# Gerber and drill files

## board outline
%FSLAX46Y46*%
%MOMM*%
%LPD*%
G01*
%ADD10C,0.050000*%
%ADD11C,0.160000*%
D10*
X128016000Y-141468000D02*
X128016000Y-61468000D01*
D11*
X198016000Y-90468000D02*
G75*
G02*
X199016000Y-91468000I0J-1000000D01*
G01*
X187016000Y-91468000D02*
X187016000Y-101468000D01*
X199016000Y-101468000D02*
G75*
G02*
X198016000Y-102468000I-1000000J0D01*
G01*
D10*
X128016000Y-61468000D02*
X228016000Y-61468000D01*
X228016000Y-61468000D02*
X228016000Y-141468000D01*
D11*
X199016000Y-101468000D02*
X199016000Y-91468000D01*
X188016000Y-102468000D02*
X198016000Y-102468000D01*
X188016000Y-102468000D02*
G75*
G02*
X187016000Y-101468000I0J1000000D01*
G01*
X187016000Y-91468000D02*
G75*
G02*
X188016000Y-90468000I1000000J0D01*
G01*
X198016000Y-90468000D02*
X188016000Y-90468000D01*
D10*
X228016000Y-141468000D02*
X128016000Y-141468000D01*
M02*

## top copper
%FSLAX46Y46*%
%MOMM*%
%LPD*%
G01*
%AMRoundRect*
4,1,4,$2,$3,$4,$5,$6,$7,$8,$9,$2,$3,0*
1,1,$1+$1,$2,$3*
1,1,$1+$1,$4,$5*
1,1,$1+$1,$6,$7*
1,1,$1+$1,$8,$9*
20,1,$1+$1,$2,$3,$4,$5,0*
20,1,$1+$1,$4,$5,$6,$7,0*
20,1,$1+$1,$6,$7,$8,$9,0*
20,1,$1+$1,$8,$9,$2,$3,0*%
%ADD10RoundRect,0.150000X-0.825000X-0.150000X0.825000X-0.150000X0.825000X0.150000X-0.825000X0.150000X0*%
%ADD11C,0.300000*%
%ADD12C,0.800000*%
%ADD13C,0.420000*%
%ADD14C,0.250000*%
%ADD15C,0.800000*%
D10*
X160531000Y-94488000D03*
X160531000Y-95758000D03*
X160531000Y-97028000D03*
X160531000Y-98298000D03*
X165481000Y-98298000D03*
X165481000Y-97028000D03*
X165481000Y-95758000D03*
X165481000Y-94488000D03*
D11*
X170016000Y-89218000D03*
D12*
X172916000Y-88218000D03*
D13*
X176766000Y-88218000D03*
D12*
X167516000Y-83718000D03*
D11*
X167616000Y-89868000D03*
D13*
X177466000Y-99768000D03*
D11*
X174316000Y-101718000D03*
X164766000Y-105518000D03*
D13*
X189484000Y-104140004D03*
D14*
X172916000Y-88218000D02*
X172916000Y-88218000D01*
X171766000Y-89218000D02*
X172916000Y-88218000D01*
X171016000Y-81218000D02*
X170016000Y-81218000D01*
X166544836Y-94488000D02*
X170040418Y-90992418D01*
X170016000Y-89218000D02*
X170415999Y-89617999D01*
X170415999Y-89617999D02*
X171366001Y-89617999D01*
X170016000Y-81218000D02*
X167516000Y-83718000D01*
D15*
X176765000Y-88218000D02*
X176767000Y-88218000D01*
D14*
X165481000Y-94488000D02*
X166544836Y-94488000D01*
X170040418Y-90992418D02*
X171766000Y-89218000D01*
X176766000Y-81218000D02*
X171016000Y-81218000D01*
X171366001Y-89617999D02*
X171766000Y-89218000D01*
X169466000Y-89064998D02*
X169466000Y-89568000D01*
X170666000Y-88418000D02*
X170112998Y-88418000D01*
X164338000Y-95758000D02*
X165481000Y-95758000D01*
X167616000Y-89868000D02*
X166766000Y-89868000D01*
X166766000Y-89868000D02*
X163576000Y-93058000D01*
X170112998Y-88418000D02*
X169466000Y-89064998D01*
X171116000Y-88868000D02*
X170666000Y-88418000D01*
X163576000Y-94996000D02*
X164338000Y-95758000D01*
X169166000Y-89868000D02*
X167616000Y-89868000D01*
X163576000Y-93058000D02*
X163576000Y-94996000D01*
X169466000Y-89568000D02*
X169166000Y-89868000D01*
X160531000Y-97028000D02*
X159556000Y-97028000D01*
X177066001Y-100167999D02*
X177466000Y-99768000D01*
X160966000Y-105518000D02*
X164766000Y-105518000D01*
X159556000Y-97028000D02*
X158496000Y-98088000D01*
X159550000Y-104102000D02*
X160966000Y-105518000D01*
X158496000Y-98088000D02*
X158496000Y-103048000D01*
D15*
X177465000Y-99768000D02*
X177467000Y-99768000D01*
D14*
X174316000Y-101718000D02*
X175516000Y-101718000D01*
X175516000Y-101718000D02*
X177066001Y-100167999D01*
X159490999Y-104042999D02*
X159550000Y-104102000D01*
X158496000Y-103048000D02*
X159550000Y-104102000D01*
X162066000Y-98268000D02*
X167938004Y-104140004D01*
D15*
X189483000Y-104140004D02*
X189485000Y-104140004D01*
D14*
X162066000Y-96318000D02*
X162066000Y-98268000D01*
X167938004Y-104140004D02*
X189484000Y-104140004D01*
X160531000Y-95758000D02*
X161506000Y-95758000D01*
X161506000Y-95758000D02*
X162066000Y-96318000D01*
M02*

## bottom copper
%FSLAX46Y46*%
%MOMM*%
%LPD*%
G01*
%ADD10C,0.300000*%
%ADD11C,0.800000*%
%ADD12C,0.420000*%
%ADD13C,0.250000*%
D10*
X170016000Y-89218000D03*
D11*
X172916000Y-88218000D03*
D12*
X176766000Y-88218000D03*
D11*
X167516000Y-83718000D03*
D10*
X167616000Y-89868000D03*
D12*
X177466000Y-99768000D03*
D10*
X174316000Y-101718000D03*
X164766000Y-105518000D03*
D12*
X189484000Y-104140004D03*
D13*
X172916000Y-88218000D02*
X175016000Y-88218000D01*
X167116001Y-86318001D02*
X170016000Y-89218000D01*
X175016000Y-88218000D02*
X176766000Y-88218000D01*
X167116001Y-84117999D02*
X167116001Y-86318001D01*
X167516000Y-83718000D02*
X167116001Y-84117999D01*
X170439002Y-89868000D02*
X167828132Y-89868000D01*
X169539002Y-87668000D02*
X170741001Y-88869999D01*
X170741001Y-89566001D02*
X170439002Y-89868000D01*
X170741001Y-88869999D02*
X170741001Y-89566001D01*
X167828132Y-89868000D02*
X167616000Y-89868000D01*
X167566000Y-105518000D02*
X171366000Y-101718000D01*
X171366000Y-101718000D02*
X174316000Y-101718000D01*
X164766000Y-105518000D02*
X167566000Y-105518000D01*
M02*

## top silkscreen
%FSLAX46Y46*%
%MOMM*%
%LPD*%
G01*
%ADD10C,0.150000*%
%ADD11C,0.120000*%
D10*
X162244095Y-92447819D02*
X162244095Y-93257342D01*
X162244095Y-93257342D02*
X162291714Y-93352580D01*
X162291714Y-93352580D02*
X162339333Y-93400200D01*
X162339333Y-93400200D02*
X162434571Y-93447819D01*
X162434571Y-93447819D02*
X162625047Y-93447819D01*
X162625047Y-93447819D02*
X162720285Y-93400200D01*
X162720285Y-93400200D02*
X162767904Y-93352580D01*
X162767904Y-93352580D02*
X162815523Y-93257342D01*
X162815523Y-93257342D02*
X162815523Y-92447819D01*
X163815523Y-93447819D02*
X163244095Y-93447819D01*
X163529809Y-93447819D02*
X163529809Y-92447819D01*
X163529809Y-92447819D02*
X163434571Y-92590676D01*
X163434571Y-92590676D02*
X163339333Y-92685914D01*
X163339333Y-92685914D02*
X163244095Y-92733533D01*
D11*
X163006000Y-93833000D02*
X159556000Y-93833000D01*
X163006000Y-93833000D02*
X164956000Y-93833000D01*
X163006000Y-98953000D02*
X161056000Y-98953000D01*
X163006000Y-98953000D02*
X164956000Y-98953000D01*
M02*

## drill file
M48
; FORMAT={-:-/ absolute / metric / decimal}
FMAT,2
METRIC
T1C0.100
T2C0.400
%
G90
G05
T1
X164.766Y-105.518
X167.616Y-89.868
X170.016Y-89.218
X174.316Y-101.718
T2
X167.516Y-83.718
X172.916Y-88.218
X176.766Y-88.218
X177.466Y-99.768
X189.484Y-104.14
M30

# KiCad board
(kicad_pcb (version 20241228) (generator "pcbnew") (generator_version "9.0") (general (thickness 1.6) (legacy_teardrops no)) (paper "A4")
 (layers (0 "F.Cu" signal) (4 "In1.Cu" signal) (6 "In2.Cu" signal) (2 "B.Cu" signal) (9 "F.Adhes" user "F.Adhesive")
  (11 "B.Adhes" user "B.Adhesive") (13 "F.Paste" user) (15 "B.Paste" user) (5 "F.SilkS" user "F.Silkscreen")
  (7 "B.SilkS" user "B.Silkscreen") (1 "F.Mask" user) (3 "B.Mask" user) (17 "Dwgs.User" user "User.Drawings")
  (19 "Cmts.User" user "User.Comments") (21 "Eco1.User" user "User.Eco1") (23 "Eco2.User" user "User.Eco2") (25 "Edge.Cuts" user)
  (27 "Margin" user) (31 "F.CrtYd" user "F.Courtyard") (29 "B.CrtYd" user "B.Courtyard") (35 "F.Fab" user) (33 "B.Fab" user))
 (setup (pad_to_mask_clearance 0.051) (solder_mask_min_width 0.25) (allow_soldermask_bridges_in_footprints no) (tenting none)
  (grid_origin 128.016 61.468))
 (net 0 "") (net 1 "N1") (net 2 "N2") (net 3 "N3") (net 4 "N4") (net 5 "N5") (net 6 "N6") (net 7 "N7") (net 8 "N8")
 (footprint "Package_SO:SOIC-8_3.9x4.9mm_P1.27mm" (layer "F.Cu") (at 163.006 96.393)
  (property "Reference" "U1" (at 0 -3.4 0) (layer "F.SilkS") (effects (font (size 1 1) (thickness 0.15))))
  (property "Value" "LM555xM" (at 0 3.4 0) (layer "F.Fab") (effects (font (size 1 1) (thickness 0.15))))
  (fp_line (start 0 -2.56) (end -3.45 -2.56) (stroke (width 0.12) (type solid)) (layer "F.SilkS"))
  (fp_line (start 0 -2.56) (end 1.95 -2.56) (stroke (width 0.12) (type solid)) (layer "F.SilkS"))
  (fp_line (start 0 2.56) (end -1.95 2.56) (stroke (width 0.12) (type solid)) (layer "F.SilkS"))
  (fp_line (start 0 2.56) (end 1.95 2.56) (stroke (width 0.12) (type solid)) (layer "F.SilkS"))
  (pad "1" smd roundrect (at -2.475 -1.905) (size 1.95 0.6) (layers "F.Cu" "F.Mask" "F.Paste") (roundrect_rratio 0.25) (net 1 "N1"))
  (pad "2" smd roundrect (at -2.475 -0.635) (size 1.95 0.6) (layers "F.Cu" "F.Mask" "F.Paste") (roundrect_rratio 0.25) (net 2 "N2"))
  (pad "3" smd roundrect (at -2.475 0.635) (size 1.95 0.6) (layers "F.Cu" "F.Mask" "F.Paste") (roundrect_rratio 0.25) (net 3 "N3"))
  (pad "4" smd roundrect (at -2.475 1.905) (size 1.95 0.6) (layers "F.Cu" "F.Mask" "F.Paste") (roundrect_rratio 0.25) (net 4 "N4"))
  (pad "5" smd roundrect (at 2.475 1.905) (size 1.95 0.6) (layers "F.Cu" "F.Mask" "F.Paste") (roundrect_rratio 0.25) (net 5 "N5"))
  (pad "6" smd roundrect (at 2.475 0.635) (size 1.95 0.6) (layers "F.Cu" "F.Mask" "F.Paste") (roundrect_rratio 0.25) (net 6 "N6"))
  (pad "7" smd roundrect (at 2.475 -0.635) (size 1.95 0.6) (layers "F.Cu" "F.Mask" "F.Paste") (roundrect_rratio 0.25) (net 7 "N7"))
  (pad "8" smd roundrect (at 2.475 -1.905) (size 1.95 0.6) (layers "F.Cu" "F.Mask" "F.Paste") (roundrect_rratio 0.25) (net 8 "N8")))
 (gr_line (start 128.016 141.468) (end 128.016 61.468) (stroke (width 0.05) (type solid)) (layer "Edge.Cuts"))
 (gr_arc (start 198.016 90.468) (mid 198.723107 90.760893) (end 199.016 91.468) (stroke (width 0.16) (type solid)) (layer "Edge.Cuts"))
 (gr_line (start 187.016 91.468) (end 187.016 101.468) (stroke (width 0.16) (type solid)) (layer "Edge.Cuts"))
 (gr_arc (start 199.016 101.468) (mid 198.723107 102.175107) (end 198.016 102.468) (stroke (width 0.16) (type solid)) (layer "Edge.Cuts"))
 (gr_line (start 128.016 61.468) (end 228.016 61.468) (stroke (width 0.05) (type solid)) (layer "Edge.Cuts"))
 (gr_line (start 228.016 61.468) (end 228.016 141.468) (stroke (width 0.05) (type solid)) (layer "Edge.Cuts"))
 (gr_line (start 199.016 101.468) (end 199.016 91.468) (stroke (width 0.16) (type solid)) (layer "Edge.Cuts"))
 (gr_line (start 188.016 102.468) (end 198.016 102.468) (stroke (width 0.16) (type solid)) (layer "Edge.Cuts"))
 (gr_arc (start 188.016 102.468) (mid 187.308893 102.175107) (end 187.016 101.468) (stroke (width 0.16) (type solid)) (layer "Edge.Cuts"))
 (gr_arc (start 187.016 91.468) (mid 187.308893 90.760893) (end 188.016 90.468) (stroke (width 0.16) (type solid)) (layer "Edge.Cuts"))
 (gr_line (start 198.016 90.468) (end 188.016 90.468) (stroke (width 0.16) (type solid)) (layer "Edge.Cuts"))
 (gr_line (start 228.016 141.468) (end 128.016 141.468) (stroke (width 0.05) (type solid)) (layer "Edge.Cuts"))
 (segment (start 172.916 88.218) (end 172.916 88.218) (width 0.25) (layer "F.Cu") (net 8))
 (segment (start 171.766 89.218) (end 172.916 88.218) (width 0.25) (layer "F.Cu") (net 8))
 (segment (start 171.016 81.218) (end 170.016 81.218) (width 0.25) (layer "F.Cu") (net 8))
 (segment (start 166.544836 94.488) (end 170.040418 90.992418) (width 0.25) (layer "F.Cu") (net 8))
 (segment (start 170.016 89.218) (end 170.415999 89.617999) (width 0.25) (layer "F.Cu") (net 8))
 (segment (start 170.415999 89.617999) (end 171.366001 89.617999) (width 0.25) (layer "F.Cu") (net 8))
 (segment (start 170.016 81.218) (end 167.516 83.718) (width 0.25) (layer "F.Cu") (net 8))
 (segment (start 176.765 88.218) (end 176.767 88.218) (width 0.8) (layer "F.Cu") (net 8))
 (segment (start 165.481 94.488) (end 166.544836 94.488) (width 0.25) (layer "F.Cu") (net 8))
 (segment (start 170.040418 90.992418) (end 171.766 89.218) (width 0.25) (layer "F.Cu") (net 8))
 (segment (start 176.766 81.218) (end 171.016 81.218) (width 0.25) (layer "F.Cu") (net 8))
 (segment (start 171.366001 89.617999) (end 171.766 89.218) (width 0.25) (layer "F.Cu") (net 8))
 (via (at 170.016 89.218) (size 0.3) (drill 0.1) (layers "F.Cu" "B.Cu") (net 8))
 (via (at 172.916 88.218) (size 0.8) (drill 0.4) (layers "F.Cu" "B.Cu") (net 8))
 (via (at 176.766 88.218) (size 0.42) (drill 0.4) (layers "F.Cu" "B.Cu") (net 8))
 (via (at 167.516 83.718) (size 0.8) (drill 0.4) (layers "F.Cu" "B.Cu") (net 8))
 (segment (start 172.916 88.218) (end 175.016 88.218) (width 0.25) (layer "B.Cu") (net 8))
 (segment (start 167.116001 86.318001) (end 170.016 89.218) (width 0.25) (layer "B.Cu") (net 8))
 (segment (start 175.016 88.218) (end 176.766 88.218) (width 0.25) (layer "B.Cu") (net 8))
 (segment (start 167.116001 84.117999) (end 167.116001 86.318001) (width 0.25) (layer "B.Cu") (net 8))
 (segment (start 167.516 83.718) (end 167.116001 84.117999) (width 0.25) (layer "B.Cu") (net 8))
 (segment (start 169.466 89.064998) (end 169.466 89.568) (width 0.25) (layer "F.Cu") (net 7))
 (segment (start 170.666 88.418) (end 170.112998 88.418) (width 0.25) (layer "F.Cu") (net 7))
 (segment (start 164.338 95.758) (end 165.481 95.758) (width 0.25) (layer "F.Cu") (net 7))
 (segment (start 167.616 89.868) (end 166.766 89.868) (width 0.25) (layer "F.Cu") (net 7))
 (segment (start 166.766 89.868) (end 163.576 93.058) (width 0.25) (layer "F.Cu") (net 7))
 (segment (start 170.112998 88.418) (end 169.466 89.064998) (width 0.25) (layer "F.Cu") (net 7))
 (segment (start 171.116 88.868) (end 170.666 88.418) (width 0.25) (layer "F.Cu") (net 7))
 (segment (start 163.576 94.996) (end 164.338 95.758) (width 0.25) (layer "F.Cu") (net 7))
 (segment (start 169.166 89.868) (end 167.616 89.868) (width 0.25) (layer "F.Cu") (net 7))
 (segment (start 163.576 93.058) (end 163.576 94.996) (width 0.25) (layer "F.Cu") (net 7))
 (segment (start 169.466 89.568) (end 169.166 89.868) (width 0.25) (layer "F.Cu") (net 7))
 (via (at 167.616 89.868) (size 0.3) (drill 0.1) (layers "F.Cu" "B.Cu") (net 7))
 (segment (start 170.439002 89.868) (end 167.828132 89.868) (width 0.25) (layer "B.Cu") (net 7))
 (segment (start 169.539002 87.668) (end 170.741001 88.869999) (width 0.25) (layer "B.Cu") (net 7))
 (segment (start 170.741001 89.566001) (end 170.439002 89.868) (width 0.25) (layer "B.Cu") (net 7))
 (segment (start 170.741001 88.869999) (end 170.741001 89.566001) (width 0.25) (layer "B.Cu") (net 7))
 (segment (start 167.828132 89.868) (end 167.616 89.868) (width 0.25) (layer "B.Cu") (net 7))
 (segment (start 160.531 97.028) (end 159.556 97.028) (width 0.25) (layer "F.Cu") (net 3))
 (segment (start 177.066001 100.167999) (end 177.466 99.768) (width 0.25) (layer "F.Cu") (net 3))
 (segment (start 160.966 105.518) (end 164.766 105.518) (width 0.25) (layer "F.Cu") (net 3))
 (segment (start 159.556 97.028) (end 158.496 98.088) (width 0.25) (layer "F.Cu") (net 3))
 (segment (start 159.55 104.102) (end 160.966 105.518) (width 0.25) (layer "F.Cu") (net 3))
 (segment (start 158.496 98.088) (end 158.496 103.048) (width 0.25) (layer "F.Cu") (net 3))
 (segment (start 177.465 99.768) (end 177.467 99.768) (width 0.8) (layer "F.Cu") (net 3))
 (segment (start 174.316 101.718) (end 175.516 101.718) (width 0.25) (layer "F.Cu") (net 3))
 (segment (start 175.516 101.718) (end 177.066001 100.167999) (width 0.25) (layer "F.Cu") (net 3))
 (segment (start 159.490999 104.042999) (end 159.55 104.102) (width 0.25) (layer "F.Cu") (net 3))
 (segment (start 158.496 103.048) (end 159.55 104.102) (width 0.25) (layer "F.Cu") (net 3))
 (via (at 177.466 99.768) (size 0.42) (drill 0.4) (layers "F.Cu" "B.Cu") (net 3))
 (via (at 174.316 101.718) (size 0.3) (drill 0.1) (layers "F.Cu" "B.Cu") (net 3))
 (via (at 164.766 105.518) (size 0.3) (drill 0.1) (layers "F.Cu" "B.Cu") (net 3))
 (segment (start 167.566 105.518) (end 171.366 101.718) (width 0.25) (layer "B.Cu") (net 3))
 (segment (start 171.366 101.718) (end 174.316 101.718) (width 0.25) (layer "B.Cu") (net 3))
 (segment (start 164.766 105.518) (end 167.566 105.518) (width 0.25) (layer "B.Cu") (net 3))
 (segment (start 162.066 98.268) (end 167.938004 104.140004) (width 0.25) (layer "F.Cu") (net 2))
 (segment (start 189.483 104.140004) (end 189.485 104.140004) (width 0.8) (layer "F.Cu") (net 2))
 (segment (start 162.066 96.318) (end 162.066 98.268) (width 0.25) (layer "F.Cu") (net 2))
 (segment (start 167.938004 104.140004) (end 189.484 104.140004) (width 0.25) (layer "F.Cu") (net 2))
 (segment (start 160.531 95.758) (end 161.506 95.758) (width 0.25) (layer "F.Cu") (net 2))
 (segment (start 161.506 95.758) (end 162.066 96.318) (width 0.25) (layer "F.Cu") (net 2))
 (via (at 189.484 104.140004) (size 0.42) (drill 0.4) (layers "F.Cu" "B.Cu") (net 2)))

